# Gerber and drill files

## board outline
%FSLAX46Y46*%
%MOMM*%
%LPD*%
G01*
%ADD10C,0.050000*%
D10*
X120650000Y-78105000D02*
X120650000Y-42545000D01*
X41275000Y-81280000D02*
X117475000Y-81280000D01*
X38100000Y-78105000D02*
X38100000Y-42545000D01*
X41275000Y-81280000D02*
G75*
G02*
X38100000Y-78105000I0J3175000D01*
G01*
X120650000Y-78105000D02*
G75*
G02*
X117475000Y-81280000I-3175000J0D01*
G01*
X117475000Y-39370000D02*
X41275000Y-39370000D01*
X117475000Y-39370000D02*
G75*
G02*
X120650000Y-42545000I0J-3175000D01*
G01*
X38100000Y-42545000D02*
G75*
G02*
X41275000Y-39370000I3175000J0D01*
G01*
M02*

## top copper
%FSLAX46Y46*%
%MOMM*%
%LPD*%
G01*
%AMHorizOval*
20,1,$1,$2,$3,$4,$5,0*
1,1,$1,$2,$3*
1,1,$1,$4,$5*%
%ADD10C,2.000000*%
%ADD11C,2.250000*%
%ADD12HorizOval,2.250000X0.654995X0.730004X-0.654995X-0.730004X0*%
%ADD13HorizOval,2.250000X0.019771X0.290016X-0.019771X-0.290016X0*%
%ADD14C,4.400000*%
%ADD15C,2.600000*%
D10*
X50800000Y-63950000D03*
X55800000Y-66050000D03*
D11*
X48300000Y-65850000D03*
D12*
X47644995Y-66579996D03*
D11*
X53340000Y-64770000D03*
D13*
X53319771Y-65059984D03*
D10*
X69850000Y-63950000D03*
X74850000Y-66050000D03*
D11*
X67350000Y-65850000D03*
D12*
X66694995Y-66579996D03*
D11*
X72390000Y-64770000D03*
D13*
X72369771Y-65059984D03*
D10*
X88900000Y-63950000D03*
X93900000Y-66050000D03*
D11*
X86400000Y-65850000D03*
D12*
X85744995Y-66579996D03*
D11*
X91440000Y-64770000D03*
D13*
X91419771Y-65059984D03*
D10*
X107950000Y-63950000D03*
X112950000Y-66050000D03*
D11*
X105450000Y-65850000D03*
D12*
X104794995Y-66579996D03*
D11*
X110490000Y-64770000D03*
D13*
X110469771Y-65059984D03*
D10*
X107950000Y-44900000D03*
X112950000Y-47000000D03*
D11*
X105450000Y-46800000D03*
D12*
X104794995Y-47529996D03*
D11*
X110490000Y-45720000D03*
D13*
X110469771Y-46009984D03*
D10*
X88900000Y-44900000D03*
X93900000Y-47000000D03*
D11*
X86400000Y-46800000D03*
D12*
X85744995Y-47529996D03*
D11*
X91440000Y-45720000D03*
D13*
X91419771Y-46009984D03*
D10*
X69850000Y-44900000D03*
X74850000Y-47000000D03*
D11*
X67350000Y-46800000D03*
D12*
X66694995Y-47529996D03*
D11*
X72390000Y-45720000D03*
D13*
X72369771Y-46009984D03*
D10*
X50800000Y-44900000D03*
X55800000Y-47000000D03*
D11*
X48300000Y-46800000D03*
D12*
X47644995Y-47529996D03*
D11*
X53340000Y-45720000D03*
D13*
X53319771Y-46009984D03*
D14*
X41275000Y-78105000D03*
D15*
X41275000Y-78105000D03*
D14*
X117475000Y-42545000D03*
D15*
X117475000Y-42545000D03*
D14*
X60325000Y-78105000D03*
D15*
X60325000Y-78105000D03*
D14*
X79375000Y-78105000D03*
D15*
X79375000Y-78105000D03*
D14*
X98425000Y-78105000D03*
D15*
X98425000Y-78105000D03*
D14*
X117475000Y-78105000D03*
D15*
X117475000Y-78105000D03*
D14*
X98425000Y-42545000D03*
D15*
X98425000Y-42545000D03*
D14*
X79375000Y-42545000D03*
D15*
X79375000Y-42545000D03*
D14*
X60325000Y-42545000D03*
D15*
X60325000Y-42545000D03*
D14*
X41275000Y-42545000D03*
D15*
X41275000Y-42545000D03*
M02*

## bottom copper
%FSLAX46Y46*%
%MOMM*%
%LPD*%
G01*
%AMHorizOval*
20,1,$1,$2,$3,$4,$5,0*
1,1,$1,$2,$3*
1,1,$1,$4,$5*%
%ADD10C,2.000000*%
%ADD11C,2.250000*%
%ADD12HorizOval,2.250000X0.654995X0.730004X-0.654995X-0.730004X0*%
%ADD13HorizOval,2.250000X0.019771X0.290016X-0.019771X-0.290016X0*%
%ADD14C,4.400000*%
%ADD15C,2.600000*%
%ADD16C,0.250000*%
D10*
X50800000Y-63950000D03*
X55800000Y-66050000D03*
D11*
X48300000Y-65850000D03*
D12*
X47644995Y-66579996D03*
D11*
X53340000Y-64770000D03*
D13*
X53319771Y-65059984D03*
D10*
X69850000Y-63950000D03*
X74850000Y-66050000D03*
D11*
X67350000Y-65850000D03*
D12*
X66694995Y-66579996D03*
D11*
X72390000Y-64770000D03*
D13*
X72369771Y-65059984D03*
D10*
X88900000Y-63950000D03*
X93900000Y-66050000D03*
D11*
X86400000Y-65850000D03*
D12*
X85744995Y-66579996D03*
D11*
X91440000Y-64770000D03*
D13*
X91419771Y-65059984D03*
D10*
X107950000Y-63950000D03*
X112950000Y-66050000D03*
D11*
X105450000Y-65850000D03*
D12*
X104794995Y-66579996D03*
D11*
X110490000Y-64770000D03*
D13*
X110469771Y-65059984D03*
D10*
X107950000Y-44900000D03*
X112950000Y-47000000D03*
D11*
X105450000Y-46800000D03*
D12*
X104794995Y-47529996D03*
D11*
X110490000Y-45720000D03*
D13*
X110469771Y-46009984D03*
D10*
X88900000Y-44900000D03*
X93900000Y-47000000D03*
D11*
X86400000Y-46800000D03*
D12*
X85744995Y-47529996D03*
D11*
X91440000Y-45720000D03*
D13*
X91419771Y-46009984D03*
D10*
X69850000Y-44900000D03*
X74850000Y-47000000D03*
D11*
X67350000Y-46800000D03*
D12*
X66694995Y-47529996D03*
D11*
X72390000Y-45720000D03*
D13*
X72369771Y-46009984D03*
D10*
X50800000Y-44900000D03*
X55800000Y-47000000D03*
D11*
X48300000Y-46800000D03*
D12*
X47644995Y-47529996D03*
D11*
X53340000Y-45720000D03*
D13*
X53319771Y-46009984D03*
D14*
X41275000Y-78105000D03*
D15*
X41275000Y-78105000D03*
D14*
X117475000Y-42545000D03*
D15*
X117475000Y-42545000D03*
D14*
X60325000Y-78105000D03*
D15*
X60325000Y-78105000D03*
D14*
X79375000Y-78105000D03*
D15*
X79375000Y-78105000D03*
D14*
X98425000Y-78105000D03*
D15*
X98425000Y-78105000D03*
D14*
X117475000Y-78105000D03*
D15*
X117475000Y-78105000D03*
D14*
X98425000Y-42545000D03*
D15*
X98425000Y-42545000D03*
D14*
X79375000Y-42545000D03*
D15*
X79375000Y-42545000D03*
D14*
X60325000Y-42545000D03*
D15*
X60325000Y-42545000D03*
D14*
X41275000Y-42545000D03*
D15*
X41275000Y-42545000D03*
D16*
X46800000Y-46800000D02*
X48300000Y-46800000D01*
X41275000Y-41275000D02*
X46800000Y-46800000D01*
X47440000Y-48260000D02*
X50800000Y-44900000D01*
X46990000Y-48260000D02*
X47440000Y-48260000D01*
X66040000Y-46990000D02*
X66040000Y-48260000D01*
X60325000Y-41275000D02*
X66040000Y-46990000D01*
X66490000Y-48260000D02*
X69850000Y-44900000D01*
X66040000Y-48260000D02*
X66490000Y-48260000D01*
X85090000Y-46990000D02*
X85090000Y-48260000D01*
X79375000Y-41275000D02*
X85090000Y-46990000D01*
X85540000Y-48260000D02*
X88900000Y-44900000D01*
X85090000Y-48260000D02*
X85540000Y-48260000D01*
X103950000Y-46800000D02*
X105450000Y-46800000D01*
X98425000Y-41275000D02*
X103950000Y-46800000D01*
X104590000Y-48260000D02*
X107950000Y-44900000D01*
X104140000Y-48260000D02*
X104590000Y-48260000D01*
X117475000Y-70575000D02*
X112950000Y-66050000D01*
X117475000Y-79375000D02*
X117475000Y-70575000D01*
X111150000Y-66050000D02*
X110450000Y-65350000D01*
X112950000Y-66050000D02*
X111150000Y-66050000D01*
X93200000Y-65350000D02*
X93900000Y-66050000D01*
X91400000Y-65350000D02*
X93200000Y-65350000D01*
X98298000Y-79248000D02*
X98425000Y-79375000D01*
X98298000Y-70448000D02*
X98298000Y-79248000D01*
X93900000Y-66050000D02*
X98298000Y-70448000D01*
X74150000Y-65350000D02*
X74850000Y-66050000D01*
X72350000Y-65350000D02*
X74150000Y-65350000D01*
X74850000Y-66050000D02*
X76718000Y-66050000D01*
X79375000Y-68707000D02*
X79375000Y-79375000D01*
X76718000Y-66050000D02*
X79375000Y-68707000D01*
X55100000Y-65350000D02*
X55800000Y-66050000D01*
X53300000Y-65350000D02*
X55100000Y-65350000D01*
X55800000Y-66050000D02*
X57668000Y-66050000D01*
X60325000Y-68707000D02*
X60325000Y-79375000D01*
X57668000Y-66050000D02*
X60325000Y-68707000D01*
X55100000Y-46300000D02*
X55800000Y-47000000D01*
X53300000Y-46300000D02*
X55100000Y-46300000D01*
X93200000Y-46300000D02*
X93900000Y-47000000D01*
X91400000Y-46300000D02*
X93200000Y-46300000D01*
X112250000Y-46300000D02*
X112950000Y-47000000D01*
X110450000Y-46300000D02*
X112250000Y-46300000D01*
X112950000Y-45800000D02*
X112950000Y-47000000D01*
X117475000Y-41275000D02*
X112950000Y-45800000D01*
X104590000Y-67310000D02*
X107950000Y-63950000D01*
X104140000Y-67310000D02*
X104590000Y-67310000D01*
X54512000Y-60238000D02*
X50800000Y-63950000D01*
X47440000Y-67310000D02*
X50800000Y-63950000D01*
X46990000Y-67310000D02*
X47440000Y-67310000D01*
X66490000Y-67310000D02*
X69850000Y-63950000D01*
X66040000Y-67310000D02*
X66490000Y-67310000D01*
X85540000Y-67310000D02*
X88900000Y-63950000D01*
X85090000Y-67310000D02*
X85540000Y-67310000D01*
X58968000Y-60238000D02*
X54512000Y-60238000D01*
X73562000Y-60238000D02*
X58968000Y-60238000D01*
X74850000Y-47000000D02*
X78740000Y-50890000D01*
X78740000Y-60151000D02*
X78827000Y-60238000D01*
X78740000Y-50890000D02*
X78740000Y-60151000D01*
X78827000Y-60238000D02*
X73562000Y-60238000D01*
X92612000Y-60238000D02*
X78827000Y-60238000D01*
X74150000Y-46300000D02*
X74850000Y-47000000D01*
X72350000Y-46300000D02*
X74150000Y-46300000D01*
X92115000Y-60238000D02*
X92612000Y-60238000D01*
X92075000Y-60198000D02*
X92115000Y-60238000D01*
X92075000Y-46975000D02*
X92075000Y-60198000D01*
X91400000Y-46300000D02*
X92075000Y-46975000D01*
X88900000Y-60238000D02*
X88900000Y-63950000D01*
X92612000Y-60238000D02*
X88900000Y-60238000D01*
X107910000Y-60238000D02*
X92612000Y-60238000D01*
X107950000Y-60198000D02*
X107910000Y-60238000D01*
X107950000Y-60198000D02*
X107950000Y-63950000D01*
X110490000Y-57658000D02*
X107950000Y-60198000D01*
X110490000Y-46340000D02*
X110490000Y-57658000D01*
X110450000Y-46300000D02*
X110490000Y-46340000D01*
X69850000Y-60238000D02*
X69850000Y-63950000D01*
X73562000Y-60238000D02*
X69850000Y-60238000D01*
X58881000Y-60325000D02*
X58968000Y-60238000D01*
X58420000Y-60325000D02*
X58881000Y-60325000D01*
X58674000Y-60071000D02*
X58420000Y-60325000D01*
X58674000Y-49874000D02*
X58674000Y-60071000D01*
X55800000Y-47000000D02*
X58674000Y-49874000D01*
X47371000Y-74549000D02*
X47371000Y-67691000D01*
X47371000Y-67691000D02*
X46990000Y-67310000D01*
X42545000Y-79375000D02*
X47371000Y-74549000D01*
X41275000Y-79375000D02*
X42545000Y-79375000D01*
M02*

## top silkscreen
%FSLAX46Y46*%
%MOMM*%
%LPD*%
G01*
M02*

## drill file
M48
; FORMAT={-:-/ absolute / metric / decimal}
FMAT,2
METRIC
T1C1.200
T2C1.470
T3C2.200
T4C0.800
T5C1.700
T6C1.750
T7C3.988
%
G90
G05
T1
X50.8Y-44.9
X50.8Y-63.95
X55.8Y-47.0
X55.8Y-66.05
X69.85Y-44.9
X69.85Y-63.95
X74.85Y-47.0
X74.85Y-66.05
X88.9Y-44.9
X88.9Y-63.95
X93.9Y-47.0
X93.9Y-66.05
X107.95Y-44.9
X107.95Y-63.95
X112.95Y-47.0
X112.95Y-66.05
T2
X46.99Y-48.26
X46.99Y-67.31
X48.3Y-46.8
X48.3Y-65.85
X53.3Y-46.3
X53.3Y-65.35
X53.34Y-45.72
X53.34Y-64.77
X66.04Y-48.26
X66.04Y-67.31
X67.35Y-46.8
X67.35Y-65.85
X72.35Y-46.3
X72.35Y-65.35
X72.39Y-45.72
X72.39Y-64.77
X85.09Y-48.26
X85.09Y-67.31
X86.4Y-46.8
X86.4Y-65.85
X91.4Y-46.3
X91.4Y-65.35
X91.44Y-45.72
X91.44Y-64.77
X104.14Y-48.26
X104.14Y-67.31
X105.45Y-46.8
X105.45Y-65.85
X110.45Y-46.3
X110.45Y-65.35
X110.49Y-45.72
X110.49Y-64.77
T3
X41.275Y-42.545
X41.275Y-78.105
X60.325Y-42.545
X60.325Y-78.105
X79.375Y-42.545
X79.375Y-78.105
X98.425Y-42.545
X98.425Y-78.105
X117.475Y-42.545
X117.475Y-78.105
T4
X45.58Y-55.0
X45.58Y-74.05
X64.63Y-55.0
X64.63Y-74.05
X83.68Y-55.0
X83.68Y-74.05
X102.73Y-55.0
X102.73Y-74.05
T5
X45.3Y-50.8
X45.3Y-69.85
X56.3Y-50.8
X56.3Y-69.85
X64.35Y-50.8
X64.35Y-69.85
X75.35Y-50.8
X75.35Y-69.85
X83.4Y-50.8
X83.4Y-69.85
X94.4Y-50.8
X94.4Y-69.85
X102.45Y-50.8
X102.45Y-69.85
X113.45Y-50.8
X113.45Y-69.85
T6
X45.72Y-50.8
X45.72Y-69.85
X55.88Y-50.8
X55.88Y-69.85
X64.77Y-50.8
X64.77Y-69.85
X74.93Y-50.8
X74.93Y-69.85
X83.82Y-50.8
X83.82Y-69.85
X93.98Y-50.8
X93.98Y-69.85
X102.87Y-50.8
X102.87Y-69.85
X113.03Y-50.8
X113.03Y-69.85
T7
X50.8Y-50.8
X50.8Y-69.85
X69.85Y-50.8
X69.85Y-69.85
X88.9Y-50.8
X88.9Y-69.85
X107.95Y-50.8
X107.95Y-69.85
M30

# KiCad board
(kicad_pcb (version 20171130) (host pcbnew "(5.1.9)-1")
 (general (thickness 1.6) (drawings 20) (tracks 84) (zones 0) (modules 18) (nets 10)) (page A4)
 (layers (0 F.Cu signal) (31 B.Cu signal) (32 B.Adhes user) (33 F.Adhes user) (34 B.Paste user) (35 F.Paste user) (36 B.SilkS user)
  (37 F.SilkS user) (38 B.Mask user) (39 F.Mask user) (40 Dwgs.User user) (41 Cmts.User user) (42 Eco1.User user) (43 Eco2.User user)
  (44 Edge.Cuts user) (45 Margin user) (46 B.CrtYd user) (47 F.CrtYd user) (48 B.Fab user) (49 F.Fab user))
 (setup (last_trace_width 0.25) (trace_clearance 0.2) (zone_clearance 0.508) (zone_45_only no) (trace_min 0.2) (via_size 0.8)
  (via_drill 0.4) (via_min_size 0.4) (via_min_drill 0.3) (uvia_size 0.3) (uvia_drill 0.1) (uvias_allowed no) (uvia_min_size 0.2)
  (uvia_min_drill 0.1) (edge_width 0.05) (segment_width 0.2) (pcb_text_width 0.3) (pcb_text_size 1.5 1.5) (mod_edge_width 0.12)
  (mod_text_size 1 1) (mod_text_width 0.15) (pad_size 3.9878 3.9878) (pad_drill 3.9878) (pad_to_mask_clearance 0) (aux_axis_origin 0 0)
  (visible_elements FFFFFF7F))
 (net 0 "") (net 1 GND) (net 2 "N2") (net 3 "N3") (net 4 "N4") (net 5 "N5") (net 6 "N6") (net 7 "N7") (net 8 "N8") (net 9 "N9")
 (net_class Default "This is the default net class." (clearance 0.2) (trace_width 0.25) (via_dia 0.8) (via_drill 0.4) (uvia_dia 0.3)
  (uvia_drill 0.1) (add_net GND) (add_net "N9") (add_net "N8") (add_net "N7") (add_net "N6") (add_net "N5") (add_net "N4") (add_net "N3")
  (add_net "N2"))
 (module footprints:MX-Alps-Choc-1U (layer F.Cu) (at 50.8 69.85)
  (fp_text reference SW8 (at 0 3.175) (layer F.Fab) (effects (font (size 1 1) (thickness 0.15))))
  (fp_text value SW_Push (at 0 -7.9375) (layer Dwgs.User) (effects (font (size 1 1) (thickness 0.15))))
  (pad "" np_thru_hole circle (at -5.22 4.2 48.1) (size 0.8 0.8) (drill 0.8) (layers *.Cu *.Mask))
  (pad "" np_thru_hole circle (at 5.5 0 48.1) (size 1.7 1.7) (drill 1.7) (layers *.Cu *.Mask))
  (pad "" np_thru_hole circle (at -5.5 0 48.1) (size 1.7 1.7) (drill 1.7) (layers *.Cu *.Mask))
  (pad 1 thru_hole circle (at 0 -5.9) (size 2 2) (drill 1.2) (layers *.Cu *.Mask) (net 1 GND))
  (pad 2 thru_hole circle (at 5 -3.8) (size 2 2) (drill 1.2) (layers *.Cu *.Mask) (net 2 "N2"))
  (pad "" np_thru_hole circle (at 5.08 0 48.0996) (size 1.75 1.75) (drill 1.75) (layers *.Cu *.Mask))
  (pad "" np_thru_hole circle (at -5.08 0 48.0996) (size 1.75 1.75) (drill 1.75) (layers *.Cu *.Mask))
  (pad 1 thru_hole circle (at -2.5 -4) (size 2.25 2.25) (drill 1.47) (layers *.Cu *.Mask) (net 1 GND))
  (pad "" np_thru_hole circle (at 0 0) (size 3.9878 3.9878) (drill 3.9878) (layers *.Cu *.Mask))
  (pad 1 thru_hole oval (at -3.81 -2.54 48.1) (size 4.211556 2.25) (drill 1.47 (offset 0.980778 0)) (layers *.Cu *.Mask) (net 1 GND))
  (pad 2 thru_hole circle (at 2.54 -5.08) (size 2.25 2.25) (drill 1.47) (layers *.Cu *.Mask) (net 2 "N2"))
  (pad 2 thru_hole oval (at 2.5 -4.5 86.1) (size 2.831378 2.25) (drill 1.47 (offset 0.290689 0)) (layers *.Cu *.Mask) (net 2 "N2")))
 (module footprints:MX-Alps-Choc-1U (layer F.Cu) (at 69.85 69.85)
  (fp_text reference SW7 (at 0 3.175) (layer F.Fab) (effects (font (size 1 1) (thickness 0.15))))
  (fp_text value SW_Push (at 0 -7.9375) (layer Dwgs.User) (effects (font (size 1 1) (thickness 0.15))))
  (pad "" np_thru_hole circle (at -5.22 4.2 48.1) (size 0.8 0.8) (drill 0.8) (layers *.Cu *.Mask))
  (pad "" np_thru_hole circle (at 5.5 0 48.1) (size 1.7 1.7) (drill 1.7) (layers *.Cu *.Mask))
  (pad "" np_thru_hole circle (at -5.5 0 48.1) (size 1.7 1.7) (drill 1.7) (layers *.Cu *.Mask))
  (pad 1 thru_hole circle (at 0 -5.9) (size 2 2) (drill 1.2) (layers *.Cu *.Mask) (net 1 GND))
  (pad 2 thru_hole circle (at 5 -3.8) (size 2 2) (drill 1.2) (layers *.Cu *.Mask) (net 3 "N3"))
  (pad "" np_thru_hole circle (at 5.08 0 48.0996) (size 1.75 1.75) (drill 1.75) (layers *.Cu *.Mask))
  (pad "" np_thru_hole circle (at -5.08 0 48.0996) (size 1.75 1.75) (drill 1.75) (layers *.Cu *.Mask))
  (pad 1 thru_hole circle (at -2.5 -4) (size 2.25 2.25) (drill 1.47) (layers *.Cu *.Mask) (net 1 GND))
  (pad "" np_thru_hole circle (at 0 0) (size 3.9878 3.9878) (drill 3.9878) (layers *.Cu *.Mask))
  (pad 1 thru_hole oval (at -3.81 -2.54 48.1) (size 4.211556 2.25) (drill 1.47 (offset 0.980778 0)) (layers *.Cu *.Mask) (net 1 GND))
  (pad 2 thru_hole circle (at 2.54 -5.08) (size 2.25 2.25) (drill 1.47) (layers *.Cu *.Mask) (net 3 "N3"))
  (pad 2 thru_hole oval (at 2.5 -4.5 86.1) (size 2.831378 2.25) (drill 1.47 (offset 0.290689 0)) (layers *.Cu *.Mask) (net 3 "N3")))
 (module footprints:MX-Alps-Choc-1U (layer F.Cu) (at 88.9 69.85)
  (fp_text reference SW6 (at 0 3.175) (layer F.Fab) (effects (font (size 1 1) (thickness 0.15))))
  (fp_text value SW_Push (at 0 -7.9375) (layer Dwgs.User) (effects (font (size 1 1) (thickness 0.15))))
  (pad "" np_thru_hole circle (at -5.22 4.2 48.1) (size 0.8 0.8) (drill 0.8) (layers *.Cu *.Mask))
  (pad "" np_thru_hole circle (at 5.5 0 48.1) (size 1.7 1.7) (drill 1.7) (layers *.Cu *.Mask))
  (pad "" np_thru_hole circle (at -5.5 0 48.1) (size 1.7 1.7) (drill 1.7) (layers *.Cu *.Mask))
  (pad 1 thru_hole circle (at 0 -5.9) (size 2 2) (drill 1.2) (layers *.Cu *.Mask) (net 1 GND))
  (pad 2 thru_hole circle (at 5 -3.8) (size 2 2) (drill 1.2) (layers *.Cu *.Mask) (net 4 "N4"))
  (pad "" np_thru_hole circle (at 5.08 0 48.0996) (size 1.75 1.75) (drill 1.75) (layers *.Cu *.Mask))
  (pad "" np_thru_hole circle (at -5.08 0 48.0996) (size 1.75 1.75) (drill 1.75) (layers *.Cu *.Mask))
  (pad 1 thru_hole circle (at -2.5 -4) (size 2.25 2.25) (drill 1.47) (layers *.Cu *.Mask) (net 1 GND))
  (pad "" np_thru_hole circle (at 0 0) (size 3.9878 3.9878) (drill 3.9878) (layers *.Cu *.Mask))
  (pad 1 thru_hole oval (at -3.81 -2.54 48.1) (size 4.211556 2.25) (drill 1.47 (offset 0.980778 0)) (layers *.Cu *.Mask) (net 1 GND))
  (pad 2 thru_hole circle (at 2.54 -5.08) (size 2.25 2.25) (drill 1.47) (layers *.Cu *.Mask) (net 4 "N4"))
  (pad 2 thru_hole oval (at 2.5 -4.5 86.1) (size 2.831378 2.25) (drill 1.47 (offset 0.290689 0)) (layers *.Cu *.Mask) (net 4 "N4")))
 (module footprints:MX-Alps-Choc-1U (layer F.Cu) (at 107.95 69.85)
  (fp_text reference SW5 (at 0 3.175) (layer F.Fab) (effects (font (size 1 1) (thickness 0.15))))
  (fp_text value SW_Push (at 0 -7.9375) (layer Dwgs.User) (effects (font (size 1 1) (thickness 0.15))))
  (pad "" np_thru_hole circle (at -5.22 4.2 48.1) (size 0.8 0.8) (drill 0.8) (layers *.Cu *.Mask))
  (pad "" np_thru_hole circle (at 5.5 0 48.1) (size 1.7 1.7) (drill 1.7) (layers *.Cu *.Mask))
  (pad "" np_thru_hole circle (at -5.5 0 48.1) (size 1.7 1.7) (drill 1.7) (layers *.Cu *.Mask))
  (pad 1 thru_hole circle (at 0 -5.9) (size 2 2) (drill 1.2) (layers *.Cu *.Mask) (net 1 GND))
  (pad 2 thru_hole circle (at 5 -3.8) (size 2 2) (drill 1.2) (layers *.Cu *.Mask) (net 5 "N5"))
  (pad "" np_thru_hole circle (at 5.08 0 48.0996) (size 1.75 1.75) (drill 1.75) (layers *.Cu *.Mask))
  (pad "" np_thru_hole circle (at -5.08 0 48.0996) (size 1.75 1.75) (drill 1.75) (layers *.Cu *.Mask))
  (pad 1 thru_hole circle (at -2.5 -4) (size 2.25 2.25) (drill 1.47) (layers *.Cu *.Mask) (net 1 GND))
  (pad "" np_thru_hole circle (at 0 0) (size 3.9878 3.9878) (drill 3.9878) (layers *.Cu *.Mask))
  (pad 1 thru_hole oval (at -3.81 -2.54 48.1) (size 4.211556 2.25) (drill 1.47 (offset 0.980778 0)) (layers *.Cu *.Mask) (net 1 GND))
  (pad 2 thru_hole circle (at 2.54 -5.08) (size 2.25 2.25) (drill 1.47) (layers *.Cu *.Mask) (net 5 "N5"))
  (pad 2 thru_hole oval (at 2.5 -4.5 86.1) (size 2.831378 2.25) (drill 1.47 (offset 0.290689 0)) (layers *.Cu *.Mask) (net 5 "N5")))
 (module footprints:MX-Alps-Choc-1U (layer F.Cu) (at 107.95 50.8)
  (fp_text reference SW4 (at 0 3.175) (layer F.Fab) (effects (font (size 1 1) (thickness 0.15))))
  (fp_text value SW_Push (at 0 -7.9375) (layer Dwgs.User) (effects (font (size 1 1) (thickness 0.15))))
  (pad "" np_thru_hole circle (at -5.22 4.2 48.1) (size 0.8 0.8) (drill 0.8) (layers *.Cu *.Mask))
  (pad "" np_thru_hole circle (at 5.5 0 48.1) (size 1.7 1.7) (drill 1.7) (layers *.Cu *.Mask))
  (pad "" np_thru_hole circle (at -5.5 0 48.1) (size 1.7 1.7) (drill 1.7) (layers *.Cu *.Mask))
  (pad 1 thru_hole circle (at 0 -5.9) (size 2 2) (drill 1.2) (layers *.Cu *.Mask) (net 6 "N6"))
  (pad 2 thru_hole circle (at 5 -3.8) (size 2 2) (drill 1.2) (layers *.Cu *.Mask) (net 1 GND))
  (pad "" np_thru_hole circle (at 5.08 0 48.0996) (size 1.75 1.75) (drill 1.75) (layers *.Cu *.Mask))
  (pad "" np_thru_hole circle (at -5.08 0 48.0996) (size 1.75 1.75) (drill 1.75) (layers *.Cu *.Mask))
  (pad 1 thru_hole circle (at -2.5 -4) (size 2.25 2.25) (drill 1.47) (layers *.Cu *.Mask) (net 6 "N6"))
  (pad "" np_thru_hole circle (at 0 0) (size 3.9878 3.9878) (drill 3.9878) (layers *.Cu *.Mask))
  (pad 1 thru_hole oval (at -3.81 -2.54 48.1) (size 4.211556 2.25) (drill 1.47 (offset 0.980778 0)) (layers *.Cu *.Mask) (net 6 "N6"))
  (pad 2 thru_hole circle (at 2.54 -5.08) (size 2.25 2.25) (drill 1.47) (layers *.Cu *.Mask) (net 1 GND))
  (pad 2 thru_hole oval (at 2.5 -4.5 86.1) (size 2.831378 2.25) (drill 1.47 (offset 0.290689 0)) (layers *.Cu *.Mask) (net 1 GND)))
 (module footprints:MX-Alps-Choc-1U (layer F.Cu) (at 88.9 50.8)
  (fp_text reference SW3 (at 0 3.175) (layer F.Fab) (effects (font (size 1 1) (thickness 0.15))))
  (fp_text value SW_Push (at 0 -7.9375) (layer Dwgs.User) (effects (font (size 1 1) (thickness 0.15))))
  (pad "" np_thru_hole circle (at -5.22 4.2 48.1) (size 0.8 0.8) (drill 0.8) (layers *.Cu *.Mask))
  (pad "" np_thru_hole circle (at 5.5 0 48.1) (size 1.7 1.7) (drill 1.7) (layers *.Cu *.Mask))
  (pad "" np_thru_hole circle (at -5.5 0 48.1) (size 1.7 1.7) (drill 1.7) (layers *.Cu *.Mask))
  (pad 1 thru_hole circle (at 0 -5.9) (size 2 2) (drill 1.2) (layers *.Cu *.Mask) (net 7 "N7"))
  (pad 2 thru_hole circle (at 5 -3.8) (size 2 2) (drill 1.2) (layers *.Cu *.Mask) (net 1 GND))
  (pad "" np_thru_hole circle (at 5.08 0 48.0996) (size 1.75 1.75) (drill 1.75) (layers *.Cu *.Mask))
  (pad "" np_thru_hole circle (at -5.08 0 48.0996) (size 1.75 1.75) (drill 1.75) (layers *.Cu *.Mask))
  (pad 1 thru_hole circle (at -2.5 -4) (size 2.25 2.25) (drill 1.47) (layers *.Cu *.Mask) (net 7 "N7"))
  (pad "" np_thru_hole circle (at 0 0) (size 3.9878 3.9878) (drill 3.9878) (layers *.Cu *.Mask))
  (pad 1 thru_hole oval (at -3.81 -2.54 48.1) (size 4.211556 2.25) (drill 1.47 (offset 0.980778 0)) (layers *.Cu *.Mask) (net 7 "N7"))
  (pad 2 thru_hole circle (at 2.54 -5.08) (size 2.25 2.25) (drill 1.47) (layers *.Cu *.Mask) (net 1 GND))
  (pad 2 thru_hole oval (at 2.5 -4.5 86.1) (size 2.831378 2.25) (drill 1.47 (offset 0.290689 0)) (layers *.Cu *.Mask) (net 1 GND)))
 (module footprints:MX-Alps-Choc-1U (layer F.Cu) (at 69.85 50.8)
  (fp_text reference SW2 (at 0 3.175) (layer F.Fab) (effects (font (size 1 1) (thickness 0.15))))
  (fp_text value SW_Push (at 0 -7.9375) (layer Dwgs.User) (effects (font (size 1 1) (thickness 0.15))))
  (pad "" np_thru_hole circle (at -5.22 4.2 48.1) (size 0.8 0.8) (drill 0.8) (layers *.Cu *.Mask))
  (pad "" np_thru_hole circle (at 5.5 0 48.1) (size 1.7 1.7) (drill 1.7) (layers *.Cu *.Mask))
  (pad "" np_thru_hole circle (at -5.5 0 48.1) (size 1.7 1.7) (drill 1.7) (layers *.Cu *.Mask))
  (pad 1 thru_hole circle (at 0 -5.9) (size 2 2) (drill 1.2) (layers *.Cu *.Mask) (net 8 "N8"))
  (pad 2 thru_hole circle (at 5 -3.8) (size 2 2) (drill 1.2) (layers *.Cu *.Mask) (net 1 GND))
  (pad "" np_thru_hole circle (at 5.08 0 48.0996) (size 1.75 1.75) (drill 1.75) (layers *.Cu *.Mask))
  (pad "" np_thru_hole circle (at -5.08 0 48.0996) (size 1.75 1.75) (drill 1.75) (layers *.Cu *.Mask))
  (pad 1 thru_hole circle (at -2.5 -4) (size 2.25 2.25) (drill 1.47) (layers *.Cu *.Mask) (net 8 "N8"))
  (pad "" np_thru_hole circle (at 0 0) (size 3.9878 3.9878) (drill 3.9878) (layers *.Cu *.Mask))
  (pad 1 thru_hole oval (at -3.81 -2.54 48.1) (size 4.211556 2.25) (drill 1.47 (offset 0.980778 0)) (layers *.Cu *.Mask) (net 8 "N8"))
  (pad 2 thru_hole circle (at 2.54 -5.08) (size 2.25 2.25) (drill 1.47) (layers *.Cu *.Mask) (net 1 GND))
  (pad 2 thru_hole oval (at 2.5 -4.5 86.1) (size 2.831378 2.25) (drill 1.47 (offset 0.290689 0)) (layers *.Cu *.Mask) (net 1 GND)))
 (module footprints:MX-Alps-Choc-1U (layer F.Cu) (at 50.8 50.8)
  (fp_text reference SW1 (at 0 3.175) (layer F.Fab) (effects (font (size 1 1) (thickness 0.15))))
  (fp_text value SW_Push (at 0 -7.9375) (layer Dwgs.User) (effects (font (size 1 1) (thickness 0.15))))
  (pad "" np_thru_hole circle (at -5.22 4.2 48.1) (size 0.8 0.8) (drill 0.8) (layers *.Cu *.Mask))
  (pad "" np_thru_hole circle (at 5.5 0 48.1) (size 1.7 1.7) (drill 1.7) (layers *.Cu *.Mask))
  (pad "" np_thru_hole circle (at -5.5 0 48.1) (size 1.7 1.7) (drill 1.7) (layers *.Cu *.Mask))
  (pad 1 thru_hole circle (at 0 -5.9) (size 2 2) (drill 1.2) (layers *.Cu *.Mask) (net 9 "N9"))
  (pad 2 thru_hole circle (at 5 -3.8) (size 2 2) (drill 1.2) (layers *.Cu *.Mask) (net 1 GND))
  (pad "" np_thru_hole circle (at 5.08 0 48.0996) (size 1.75 1.75) (drill 1.75) (layers *.Cu *.Mask))
  (pad "" np_thru_hole circle (at -5.08 0 48.0996) (size 1.75 1.75) (drill 1.75) (layers *.Cu *.Mask))
  (pad 1 thru_hole circle (at -2.5 -4) (size 2.25 2.25) (drill 1.47) (layers *.Cu *.Mask) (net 9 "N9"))
  (pad "" np_thru_hole circle (at 0 0) (size 3.9878 3.9878) (drill 3.9878) (layers *.Cu *.Mask))
  (pad 1 thru_hole oval (at -3.81 -2.54 48.1) (size 4.211556 2.25) (drill 1.47 (offset 0.980778 0)) (layers *.Cu *.Mask) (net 9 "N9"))
  (pad 2 thru_hole circle (at 2.54 -5.08) (size 2.25 2.25) (drill 1.47) (layers *.Cu *.Mask) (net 1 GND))
  (pad 2 thru_hole oval (at 2.5 -4.5 86.1) (size 2.831378 2.25) (drill 1.47 (offset 0.290689 0)) (layers *.Cu *.Mask) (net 1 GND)))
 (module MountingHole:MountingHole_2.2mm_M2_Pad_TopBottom (layer F.Cu) (at 41.275 78.105)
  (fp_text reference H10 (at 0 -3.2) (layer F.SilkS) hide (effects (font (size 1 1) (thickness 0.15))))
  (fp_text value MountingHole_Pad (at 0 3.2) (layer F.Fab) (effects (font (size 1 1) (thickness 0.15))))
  (pad 1 connect circle (at 0 0) (size 4.4 4.4) (layers B.Cu B.Mask) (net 1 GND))
  (pad 1 connect circle (at 0 0) (size 4.4 4.4) (layers F.Cu F.Mask) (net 1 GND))
  (pad 1 thru_hole circle (at 0 0) (size 2.6 2.6) (drill 2.2) (layers *.Cu *.Mask) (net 1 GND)))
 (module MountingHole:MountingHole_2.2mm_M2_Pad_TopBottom (layer F.Cu) (at 117.475 42.545)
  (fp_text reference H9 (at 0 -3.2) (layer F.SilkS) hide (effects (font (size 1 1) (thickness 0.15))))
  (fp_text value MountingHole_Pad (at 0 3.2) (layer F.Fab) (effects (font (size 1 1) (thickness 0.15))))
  (pad 1 connect circle (at 0 0) (size 4.4 4.4) (layers B.Cu B.Mask) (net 1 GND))
  (pad 1 connect circle (at 0 0) (size 4.4 4.4) (layers F.Cu F.Mask) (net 1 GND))
  (pad 1 thru_hole circle (at 0 0) (size 2.6 2.6) (drill 2.2) (layers *.Cu *.Mask) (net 1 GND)))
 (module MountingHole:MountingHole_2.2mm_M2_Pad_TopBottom (layer F.Cu) (at 60.325 78.105)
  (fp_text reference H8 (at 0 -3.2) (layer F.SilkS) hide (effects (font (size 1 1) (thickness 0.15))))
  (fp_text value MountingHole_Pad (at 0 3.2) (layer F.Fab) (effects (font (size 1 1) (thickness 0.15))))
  (pad 1 connect circle (at 0 0) (size 4.4 4.4) (layers B.Cu B.Mask) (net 2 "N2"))
  (pad 1 connect circle (at 0 0) (size 4.4 4.4) (layers F.Cu F.Mask) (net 2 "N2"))
  (pad 1 thru_hole circle (at 0 0) (size 2.6 2.6) (drill 2.2) (layers *.Cu *.Mask) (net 2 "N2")))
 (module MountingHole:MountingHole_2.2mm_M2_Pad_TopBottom (layer F.Cu) (at 79.375 78.105)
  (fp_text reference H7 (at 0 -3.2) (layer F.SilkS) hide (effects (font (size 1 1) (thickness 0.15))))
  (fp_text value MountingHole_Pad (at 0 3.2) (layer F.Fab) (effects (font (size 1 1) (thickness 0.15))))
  (pad 1 connect circle (at 0 0) (size 4.4 4.4) (layers B.Cu B.Mask) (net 3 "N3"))
  (pad 1 connect circle (at 0 0) (size 4.4 4.4) (layers F.Cu F.Mask) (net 3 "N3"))
  (pad 1 thru_hole circle (at 0 0) (size 2.6 2.6) (drill 2.2) (layers *.Cu *.Mask) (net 3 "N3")))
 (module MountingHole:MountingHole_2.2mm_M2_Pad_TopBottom (layer F.Cu) (at 98.425 78.105)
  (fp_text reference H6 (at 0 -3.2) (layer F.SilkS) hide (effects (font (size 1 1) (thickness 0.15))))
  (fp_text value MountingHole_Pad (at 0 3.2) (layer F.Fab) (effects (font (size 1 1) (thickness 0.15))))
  (pad 1 connect circle (at 0 0) (size 4.4 4.4) (layers B.Cu B.Mask) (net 4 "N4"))
  (pad 1 connect circle (at 0 0) (size 4.4 4.4) (layers F.Cu F.Mask) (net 4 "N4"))
  (pad 1 thru_hole circle (at 0 0) (size 2.6 2.6) (drill 2.2) (layers *.Cu *.Mask) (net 4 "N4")))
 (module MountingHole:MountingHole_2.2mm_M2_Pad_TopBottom (layer F.Cu) (at 117.475 78.105)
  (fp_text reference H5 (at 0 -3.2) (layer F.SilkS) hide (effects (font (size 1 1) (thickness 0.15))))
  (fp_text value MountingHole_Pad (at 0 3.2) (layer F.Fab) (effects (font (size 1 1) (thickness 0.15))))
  (pad 1 connect circle (at 0 0) (size 4.4 4.4) (layers B.Cu B.Mask) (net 5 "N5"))
  (pad 1 connect circle (at 0 0) (size 4.4 4.4) (layers F.Cu F.Mask) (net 5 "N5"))
  (pad 1 thru_hole circle (at 0 0) (size 2.6 2.6) (drill 2.2) (layers *.Cu *.Mask) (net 5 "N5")))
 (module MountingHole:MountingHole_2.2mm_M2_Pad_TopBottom (layer F.Cu) (at 98.425 42.545)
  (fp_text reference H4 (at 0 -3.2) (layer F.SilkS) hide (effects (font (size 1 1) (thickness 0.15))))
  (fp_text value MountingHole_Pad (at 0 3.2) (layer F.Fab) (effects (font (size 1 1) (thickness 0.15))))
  (pad 1 connect circle (at 0 0) (size 4.4 4.4) (layers B.Cu B.Mask) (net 6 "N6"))
  (pad 1 connect circle (at 0 0) (size 4.4 4.4) (layers F.Cu F.Mask) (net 6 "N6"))
  (pad 1 thru_hole circle (at 0 0) (size 2.6 2.6) (drill 2.2) (layers *.Cu *.Mask) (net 6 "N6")))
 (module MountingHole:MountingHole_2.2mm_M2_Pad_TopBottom (layer F.Cu) (at 79.375 42.545)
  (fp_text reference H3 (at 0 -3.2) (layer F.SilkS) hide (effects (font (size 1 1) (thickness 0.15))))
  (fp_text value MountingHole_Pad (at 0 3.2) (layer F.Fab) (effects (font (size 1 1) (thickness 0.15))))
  (pad 1 connect circle (at 0 0) (size 4.4 4.4) (layers B.Cu B.Mask) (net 7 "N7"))
  (pad 1 connect circle (at 0 0) (size 4.4 4.4) (layers F.Cu F.Mask) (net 7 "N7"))
  (pad 1 thru_hole circle (at 0 0) (size 2.6 2.6) (drill 2.2) (layers *.Cu *.Mask) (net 7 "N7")))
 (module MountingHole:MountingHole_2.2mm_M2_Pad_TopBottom (layer F.Cu) (at 60.325 42.545)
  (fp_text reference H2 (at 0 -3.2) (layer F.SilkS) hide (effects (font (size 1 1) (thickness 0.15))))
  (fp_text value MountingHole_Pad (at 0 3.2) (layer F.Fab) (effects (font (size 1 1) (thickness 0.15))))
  (pad 1 connect circle (at 0 0) (size 4.4 4.4) (layers B.Cu B.Mask) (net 8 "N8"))
  (pad 1 connect circle (at 0 0) (size 4.4 4.4) (layers F.Cu F.Mask) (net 8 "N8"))
  (pad 1 thru_hole circle (at 0 0) (size 2.6 2.6) (drill 2.2) (layers *.Cu *.Mask) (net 8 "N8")))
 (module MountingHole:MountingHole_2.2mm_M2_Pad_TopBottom (layer F.Cu) (at 41.275 42.545)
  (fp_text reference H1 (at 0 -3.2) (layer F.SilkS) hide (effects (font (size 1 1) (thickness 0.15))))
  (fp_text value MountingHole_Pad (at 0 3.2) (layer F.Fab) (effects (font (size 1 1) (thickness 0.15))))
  (pad 1 connect circle (at 0 0) (size 4.4 4.4) (layers B.Cu B.Mask) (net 9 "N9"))
  (pad 1 connect circle (at 0 0) (size 4.4 4.4) (layers F.Cu F.Mask) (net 9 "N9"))
  (pad 1 thru_hole circle (at 0 0) (size 2.6 2.6) (drill 2.2) (layers *.Cu *.Mask) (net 9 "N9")))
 (gr_line (start 120.65 78.105) (end 120.65 42.545) (layer Edge.Cuts) (width 0.05))
 (gr_line (start 41.275 81.28) (end 117.475 81.28) (layer Edge.Cuts) (width 0.05))
 (gr_line (start 38.1 78.105) (end 38.1 42.545) (layer Edge.Cuts) (width 0.05))
 (gr_arc (start 41.275 78.105) (end 38.1 78.105) (angle -90) (layer Edge.Cuts) (width 0.05))
 (gr_arc (start 117.475 78.105) (end 117.475 81.28) (angle -90) (layer Edge.Cuts) (width 0.05))
 (gr_line (start 117.475 39.37) (end 41.275 39.37) (layer Edge.Cuts) (width 0.05))
 (gr_arc (start 117.475 42.545) (end 120.65 42.545) (angle -90) (layer Edge.Cuts) (width 0.05))
 (gr_arc (start 41.275 42.545) (end 41.275 39.37) (angle -90) (layer Edge.Cuts) (width 0.05))
 (segment (start 46.8 46.8) (end 48.3 46.8) (width 0.25) (layer B.Cu) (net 9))
 (segment (start 41.275 41.275) (end 46.8 46.8) (width 0.25) (layer B.Cu) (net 9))
 (segment (start 47.44 48.26) (end 50.8 44.9) (width 0.25) (layer B.Cu) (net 9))
 (segment (start 46.99 48.26) (end 47.44 48.26) (width 0.25) (layer B.Cu) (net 9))
 (segment (start 66.04 46.99) (end 66.04 48.26) (width 0.25) (layer B.Cu) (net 8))
 (segment (start 60.325 41.275) (end 66.04 46.99) (width 0.25) (layer B.Cu) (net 8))
 (segment (start 66.49 48.26) (end 69.85 44.9) (width 0.25) (layer B.Cu) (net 8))
 (segment (start 66.04 48.26) (end 66.49 48.26) (width 0.25) (layer B.Cu) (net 8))
 (segment (start 85.09 46.99) (end 85.09 48.26) (width 0.25) (layer B.Cu) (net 7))
 (segment (start 79.375 41.275) (end 85.09 46.99) (width 0.25) (layer B.Cu) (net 7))
 (segment (start 85.54 48.26) (end 88.9 44.9) (width 0.25) (layer B.Cu) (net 7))
 (segment (start 85.09 48.26) (end 85.54 48.26) (width 0.25) (layer B.Cu) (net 7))
 (segment (start 103.95 46.8) (end 105.45 46.8) (width 0.25) (layer B.Cu) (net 6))
 (segment (start 98.425 41.275) (end 103.95 46.8) (width 0.25) (layer B.Cu) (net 6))
 (segment (start 104.59 48.26) (end 107.95 44.9) (width 0.25) (layer B.Cu) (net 6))
 (segment (start 104.14 48.26) (end 104.59 48.26) (width 0.25) (layer B.Cu) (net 6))
 (segment (start 117.475 70.575) (end 112.95 66.05) (width 0.25) (layer B.Cu) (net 5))
 (segment (start 117.475 79.375) (end 117.475 70.575) (width 0.25) (layer B.Cu) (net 5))
 (segment (start 111.15 66.05) (end 110.45 65.35) (width 0.25) (layer B.Cu) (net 5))
 (segment (start 112.95 66.05) (end 111.15 66.05) (width 0.25) (layer B.Cu) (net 5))
 (segment (start 93.2 65.35) (end 93.9 66.05) (width 0.25) (layer B.Cu) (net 4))
 (segment (start 91.4 65.35) (end 93.2 65.35) (width 0.25) (layer B.Cu) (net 4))
 (segment (start 98.298 79.248) (end 98.425 79.375) (width 0.25) (layer B.Cu) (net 4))
 (segment (start 98.298 70.448) (end 98.298 79.248) (width 0.25) (layer B.Cu) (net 4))
 (segment (start 93.9 66.05) (end 98.298 70.448) (width 0.25) (layer B.Cu) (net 4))
 (segment (start 74.15 65.35) (end 74.85 66.05) (width 0.25) (layer B.Cu) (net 3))
 (segment (start 72.35 65.35) (end 74.15 65.35) (width 0.25) (layer B.Cu) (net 3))
 (segment (start 74.85 66.05) (end 76.718 66.05) (width 0.25) (layer B.Cu) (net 3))
 (segment (start 79.375 68.707) (end 79.375 79.375) (width 0.25) (layer B.Cu) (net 3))
 (segment (start 76.718 66.05) (end 79.375 68.707) (width 0.25) (layer B.Cu) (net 3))
 (segment (start 55.1 65.35) (end 55.8 66.05) (width 0.25) (layer B.Cu) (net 2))
 (segment (start 53.3 65.35) (end 55.1 65.35) (width 0.25) (layer B.Cu) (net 2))
 (segment (start 55.8 66.05) (end 57.668 66.05) (width 0.25) (layer B.Cu) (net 2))
 (segment (start 60.325 68.707) (end 60.325 79.375) (width 0.25) (layer B.Cu) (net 2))
 (segment (start 57.668 66.05) (end 60.325 68.707) (width 0.25) (layer B.Cu) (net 2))
 (segment (start 55.1 46.3) (end 55.8 47) (width 0.25) (layer B.Cu) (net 1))
 (segment (start 53.3 46.3) (end 55.1 46.3) (width 0.25) (layer B.Cu) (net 1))
 (segment (start 93.2 46.3) (end 93.9 47) (width 0.25) (layer B.Cu) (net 1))
 (segment (start 91.4 46.3) (end 93.2 46.3) (width 0.25) (layer B.Cu) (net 1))
 (segment (start 112.25 46.3) (end 112.95 47) (width 0.25) (layer B.Cu) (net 1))
 (segment (start 110.45 46.3) (end 112.25 46.3) (width 0.25) (layer B.Cu) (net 1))
 (segment (start 112.95 45.8) (end 112.95 47) (width 0.25) (layer B.Cu) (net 1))
 (segment (start 117.475 41.275) (end 112.95 45.8) (width 0.25) (layer B.Cu) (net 1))
 (segment (start 104.59 67.31) (end 107.95 63.95) (width 0.25) (layer B.Cu) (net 1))
 (segment (start 104.14 67.31) (end 104.59 67.31) (width 0.25) (layer B.Cu) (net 1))
 (segment (start 54.512 60.238) (end 50.8 63.95) (width 0.25) (layer B.Cu) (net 1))
 (segment (start 47.44 67.31) (end 50.8 63.95) (width 0.25) (layer B.Cu) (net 1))
 (segment (start 46.99 67.31) (end 47.44 67.31) (width 0.25) (layer B.Cu) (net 1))
 (segment (start 66.49 67.31) (end 69.85 63.95) (width 0.25) (layer B.Cu) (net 1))
 (segment (start 66.04 67.31) (end 66.49 67.31) (width 0.25) (layer B.Cu) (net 1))
 (segment (start 85.54 67.31) (end 88.9 63.95) (width 0.25) (layer B.Cu) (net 1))
 (segment (start 85.09 67.31) (end 85.54 67.31) (width 0.25) (layer B.Cu) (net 1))
 (segment (start 58.968 60.238) (end 54.512 60.238) (width 0.25) (layer B.Cu) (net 1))
 (segment (start 73.562 60.238) (end 58.968 60.238) (width 0.25) (layer B.Cu) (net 1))
 (segment (start 74.85 47) (end 78.74 50.89) (width 0.25) (layer B.Cu) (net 1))
 (segment (start 78.74 60.151) (end 78.827 60.238) (width 0.25) (layer B.Cu) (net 1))
 (segment (start 78.74 50.89) (end 78.74 60.151) (width 0.25) (layer B.Cu) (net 1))
 (segment (start 78.827 60.238) (end 73.562 60.238) (width 0.25) (layer B.Cu) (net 1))
 (segment (start 92.612 60.238) (end 78.827 60.238) (width 0.25) (layer B.Cu) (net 1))
 (segment (start 74.15 46.3) (end 74.85 47) (width 0.25) (layer B.Cu) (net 1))
 (segment (start 72.35 46.3) (end 74.15 46.3) (width 0.25) (layer B.Cu) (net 1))
 (segment (start 92.115 60.238) (end 92.612 60.238) (width 0.25) (layer B.Cu) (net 1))
 (segment (start 92.075 60.198) (end 92.115 60.238) (width 0.25) (layer B.Cu) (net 1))
 (segment (start 92.075 46.975) (end 92.075 60.198) (width 0.25) (layer B.Cu) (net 1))
 (segment (start 91.4 46.3) (end 92.075 46.975) (width 0.25) (layer B.Cu) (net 1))
 (segment (start 88.9 60.238) (end 88.9 63.95) (width 0.25) (layer B.Cu) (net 1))
 (segment (start 92.612 60.238) (end 88.9 60.238) (width 0.25) (layer B.Cu) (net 1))
 (segment (start 107.91 60.238) (end 92.612 60.238) (width 0.25) (layer B.Cu) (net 1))
 (segment (start 107.95 60.198) (end 107.91 60.238) (width 0.25) (layer B.Cu) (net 1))
 (segment (start 107.95 60.198) (end 107.95 63.95) (width 0.25) (layer B.Cu) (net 1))
 (segment (start 110.49 57.658) (end 107.95 60.198) (width 0.25) (layer B.Cu) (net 1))
 (segment (start 110.49 46.34) (end 110.49 57.658) (width 0.25) (layer B.Cu) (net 1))
 (segment (start 110.45 46.3) (end 110.49 46.34) (width 0.25) (layer B.Cu) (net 1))
 (segment (start 69.85 60.238) (end 69.85 63.95) (width 0.25) (layer B.Cu) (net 1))
 (segment (start 73.562 60.238) (end 69.85 60.238) (width 0.25) (layer B.Cu) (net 1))
 (segment (start 58.881 60.325) (end 58.968 60.238) (width 0.25) (layer B.Cu) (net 1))
 (segment (start 58.42 60.325) (end 58.881 60.325) (width 0.25) (layer B.Cu) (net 1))
 (segment (start 58.674 60.071) (end 58.42 60.325) (width 0.25) (layer B.Cu) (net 1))
 (segment (start 58.674 49.874) (end 58.674 60.071) (width 0.25) (layer B.Cu) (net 1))
 (segment (start 55.8 47) (end 58.674 49.874) (width 0.25) (layer B.Cu) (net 1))
 (segment (start 47.371 74.549) (end 47.371 67.691) (width 0.25) (layer B.Cu) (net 1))
 (segment (start 47.371 67.691) (end 46.99 67.31) (width 0.25) (layer B.Cu) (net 1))
 (segment (start 42.545 79.375) (end 47.371 74.549) (width 0.25) (layer B.Cu) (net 1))
 (segment (start 41.275 79.375) (end 42.545 79.375) (width 0.25) (layer B.Cu) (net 1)))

